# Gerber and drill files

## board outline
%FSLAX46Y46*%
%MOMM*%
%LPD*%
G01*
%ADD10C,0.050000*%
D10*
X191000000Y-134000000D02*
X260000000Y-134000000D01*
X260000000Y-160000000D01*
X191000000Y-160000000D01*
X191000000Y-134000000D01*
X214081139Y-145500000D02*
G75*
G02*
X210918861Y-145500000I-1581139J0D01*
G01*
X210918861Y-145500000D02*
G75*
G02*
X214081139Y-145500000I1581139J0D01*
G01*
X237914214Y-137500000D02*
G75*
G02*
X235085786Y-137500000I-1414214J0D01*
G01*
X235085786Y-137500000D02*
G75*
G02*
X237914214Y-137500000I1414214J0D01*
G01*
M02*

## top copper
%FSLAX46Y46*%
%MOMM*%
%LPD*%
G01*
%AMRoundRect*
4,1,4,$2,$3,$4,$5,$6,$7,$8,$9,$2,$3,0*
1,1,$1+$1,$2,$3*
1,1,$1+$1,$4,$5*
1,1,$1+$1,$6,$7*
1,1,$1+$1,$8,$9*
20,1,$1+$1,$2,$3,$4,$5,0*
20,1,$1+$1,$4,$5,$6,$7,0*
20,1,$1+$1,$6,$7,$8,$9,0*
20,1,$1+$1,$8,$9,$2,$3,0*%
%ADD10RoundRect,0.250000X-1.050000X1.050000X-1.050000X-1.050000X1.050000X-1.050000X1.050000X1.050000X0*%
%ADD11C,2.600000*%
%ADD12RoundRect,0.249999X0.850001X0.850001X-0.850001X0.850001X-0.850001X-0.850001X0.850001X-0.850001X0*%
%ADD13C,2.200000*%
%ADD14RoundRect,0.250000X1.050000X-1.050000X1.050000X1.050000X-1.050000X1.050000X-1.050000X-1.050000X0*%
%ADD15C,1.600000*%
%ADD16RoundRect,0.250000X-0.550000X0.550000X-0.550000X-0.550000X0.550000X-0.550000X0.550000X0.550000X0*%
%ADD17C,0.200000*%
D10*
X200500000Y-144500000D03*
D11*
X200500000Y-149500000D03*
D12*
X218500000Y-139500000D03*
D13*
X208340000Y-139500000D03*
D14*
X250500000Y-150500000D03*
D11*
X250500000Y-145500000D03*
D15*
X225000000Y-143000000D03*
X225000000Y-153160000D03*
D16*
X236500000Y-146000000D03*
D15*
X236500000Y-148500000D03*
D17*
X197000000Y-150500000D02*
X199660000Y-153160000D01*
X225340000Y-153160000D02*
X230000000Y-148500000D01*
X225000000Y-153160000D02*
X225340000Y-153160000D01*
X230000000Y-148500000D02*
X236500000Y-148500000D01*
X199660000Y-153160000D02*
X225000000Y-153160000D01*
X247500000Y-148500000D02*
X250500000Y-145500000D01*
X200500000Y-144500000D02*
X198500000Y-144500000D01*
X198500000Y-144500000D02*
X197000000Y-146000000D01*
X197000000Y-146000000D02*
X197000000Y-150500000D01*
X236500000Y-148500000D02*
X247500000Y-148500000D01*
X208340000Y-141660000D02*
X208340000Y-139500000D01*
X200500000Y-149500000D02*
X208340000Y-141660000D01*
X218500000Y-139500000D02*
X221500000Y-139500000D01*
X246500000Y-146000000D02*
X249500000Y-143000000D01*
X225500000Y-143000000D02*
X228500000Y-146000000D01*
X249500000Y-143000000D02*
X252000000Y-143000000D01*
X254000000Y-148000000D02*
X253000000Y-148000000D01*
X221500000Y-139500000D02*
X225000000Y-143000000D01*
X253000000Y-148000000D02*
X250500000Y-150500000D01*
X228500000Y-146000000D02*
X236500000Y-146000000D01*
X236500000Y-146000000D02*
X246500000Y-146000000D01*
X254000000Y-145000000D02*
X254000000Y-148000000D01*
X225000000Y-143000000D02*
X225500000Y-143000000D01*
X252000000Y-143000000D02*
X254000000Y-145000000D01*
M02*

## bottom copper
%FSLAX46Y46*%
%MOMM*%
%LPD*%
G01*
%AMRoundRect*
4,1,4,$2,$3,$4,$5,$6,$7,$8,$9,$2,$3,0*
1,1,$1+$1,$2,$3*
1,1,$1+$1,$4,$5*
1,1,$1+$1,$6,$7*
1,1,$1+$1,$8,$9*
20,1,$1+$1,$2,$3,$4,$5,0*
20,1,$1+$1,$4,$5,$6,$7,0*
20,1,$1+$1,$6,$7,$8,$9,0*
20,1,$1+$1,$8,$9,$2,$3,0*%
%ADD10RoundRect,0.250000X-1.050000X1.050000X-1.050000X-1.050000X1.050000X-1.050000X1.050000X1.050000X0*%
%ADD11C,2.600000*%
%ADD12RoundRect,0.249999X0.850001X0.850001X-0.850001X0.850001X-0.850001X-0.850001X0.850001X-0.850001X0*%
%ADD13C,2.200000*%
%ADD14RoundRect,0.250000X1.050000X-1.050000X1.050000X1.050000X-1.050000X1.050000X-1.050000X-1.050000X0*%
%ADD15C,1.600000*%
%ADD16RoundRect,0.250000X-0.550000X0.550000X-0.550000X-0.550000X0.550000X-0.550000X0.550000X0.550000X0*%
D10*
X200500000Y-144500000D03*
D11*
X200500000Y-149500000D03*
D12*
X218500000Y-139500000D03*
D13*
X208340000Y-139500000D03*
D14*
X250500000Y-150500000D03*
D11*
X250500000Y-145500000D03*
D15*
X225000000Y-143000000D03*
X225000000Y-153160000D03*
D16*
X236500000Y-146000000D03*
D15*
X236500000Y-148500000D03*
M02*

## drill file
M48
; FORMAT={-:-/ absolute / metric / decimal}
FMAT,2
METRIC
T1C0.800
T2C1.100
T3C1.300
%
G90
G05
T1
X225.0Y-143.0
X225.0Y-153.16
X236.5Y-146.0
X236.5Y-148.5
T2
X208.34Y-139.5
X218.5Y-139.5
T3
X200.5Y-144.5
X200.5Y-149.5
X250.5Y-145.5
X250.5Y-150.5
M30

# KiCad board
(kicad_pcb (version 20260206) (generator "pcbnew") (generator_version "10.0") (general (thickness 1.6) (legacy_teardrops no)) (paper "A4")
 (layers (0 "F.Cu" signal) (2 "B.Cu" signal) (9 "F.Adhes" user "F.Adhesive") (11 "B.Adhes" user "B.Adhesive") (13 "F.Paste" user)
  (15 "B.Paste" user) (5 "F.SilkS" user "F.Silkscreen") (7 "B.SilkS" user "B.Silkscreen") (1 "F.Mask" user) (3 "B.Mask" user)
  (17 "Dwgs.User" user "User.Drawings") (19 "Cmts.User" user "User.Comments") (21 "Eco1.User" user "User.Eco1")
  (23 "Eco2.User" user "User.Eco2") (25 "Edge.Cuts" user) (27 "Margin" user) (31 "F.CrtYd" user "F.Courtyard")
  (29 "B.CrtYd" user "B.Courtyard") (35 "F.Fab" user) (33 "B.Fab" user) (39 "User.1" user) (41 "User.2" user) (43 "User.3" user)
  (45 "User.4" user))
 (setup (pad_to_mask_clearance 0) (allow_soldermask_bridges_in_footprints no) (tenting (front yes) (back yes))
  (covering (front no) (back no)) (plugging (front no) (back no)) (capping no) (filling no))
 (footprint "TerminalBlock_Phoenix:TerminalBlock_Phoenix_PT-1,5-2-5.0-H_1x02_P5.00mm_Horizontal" (layer "F.Cu") (at 200.5 144.5 -90)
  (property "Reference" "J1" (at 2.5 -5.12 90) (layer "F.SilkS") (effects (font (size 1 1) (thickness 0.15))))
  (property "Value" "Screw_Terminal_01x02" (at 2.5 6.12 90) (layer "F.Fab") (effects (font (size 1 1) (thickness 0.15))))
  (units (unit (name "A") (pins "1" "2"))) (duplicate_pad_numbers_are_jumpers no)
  (pad "1" thru_hole roundrect (at 0 0 270) (size 2.6 2.6) (drill 1.3) (layers "*.Cu" "*.Mask") (remove_unused_layers no)
   (roundrect_rratio 0.096154) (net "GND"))
  (pad "2" thru_hole circle (at 5 0 270) (size 2.6 2.6) (drill 1.3) (layers "*.Cu" "*.Mask") (remove_unused_layers no) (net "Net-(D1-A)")))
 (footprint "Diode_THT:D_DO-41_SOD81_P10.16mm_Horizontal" (layer "F.Cu") (at 218.5 139.5 180)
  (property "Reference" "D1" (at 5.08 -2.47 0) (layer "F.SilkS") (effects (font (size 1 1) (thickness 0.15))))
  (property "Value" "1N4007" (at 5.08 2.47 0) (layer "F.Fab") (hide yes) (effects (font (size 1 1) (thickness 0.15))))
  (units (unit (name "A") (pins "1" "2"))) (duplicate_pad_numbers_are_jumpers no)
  (pad "1" thru_hole roundrect (at 0 0 180) (size 2.2 2.2) (drill 1.1) (layers "*.Cu" "*.Mask") (remove_unused_layers no)
   (roundrect_rratio 0.113636) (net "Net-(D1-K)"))
  (pad "2" thru_hole circle (at 10.16 0 180) (size 2.2 2.2) (drill 1.1) (layers "*.Cu" "*.Mask") (remove_unused_layers no)
   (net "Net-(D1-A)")))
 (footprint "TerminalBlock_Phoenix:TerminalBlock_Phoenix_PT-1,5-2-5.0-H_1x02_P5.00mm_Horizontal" (layer "F.Cu") (at 250.5 150.5 90)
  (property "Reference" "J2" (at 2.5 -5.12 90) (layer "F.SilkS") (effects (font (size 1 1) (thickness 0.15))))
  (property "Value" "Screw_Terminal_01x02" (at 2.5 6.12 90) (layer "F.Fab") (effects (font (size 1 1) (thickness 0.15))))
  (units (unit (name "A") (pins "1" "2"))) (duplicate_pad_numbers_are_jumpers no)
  (pad "1" thru_hole roundrect (at 0 0 90) (size 2.6 2.6) (drill 1.3) (layers "*.Cu" "*.Mask") (remove_unused_layers no)
   (roundrect_rratio 0.096154) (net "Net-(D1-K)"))
  (pad "2" thru_hole circle (at 5 0 90) (size 2.6 2.6) (drill 1.3) (layers "*.Cu" "*.Mask") (remove_unused_layers no) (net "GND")))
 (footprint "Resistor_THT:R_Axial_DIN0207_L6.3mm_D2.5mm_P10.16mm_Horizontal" (layer "F.Cu") (at 225 143 -90)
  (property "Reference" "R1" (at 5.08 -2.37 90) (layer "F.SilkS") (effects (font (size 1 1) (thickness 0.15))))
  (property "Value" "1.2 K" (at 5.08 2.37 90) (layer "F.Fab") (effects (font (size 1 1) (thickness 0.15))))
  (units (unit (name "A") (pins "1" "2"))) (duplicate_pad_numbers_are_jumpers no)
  (pad "1" thru_hole circle (at 0 0 270) (size 1.6 1.6) (drill 0.8) (layers "*.Cu" "*.Mask") (remove_unused_layers no) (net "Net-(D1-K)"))
  (pad "2" thru_hole circle (at 10.16 0 270) (size 1.6 1.6) (drill 0.8) (layers "*.Cu" "*.Mask") (remove_unused_layers no) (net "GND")))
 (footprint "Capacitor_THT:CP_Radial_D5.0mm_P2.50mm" (layer "F.Cu") (at 236.5 146 -90)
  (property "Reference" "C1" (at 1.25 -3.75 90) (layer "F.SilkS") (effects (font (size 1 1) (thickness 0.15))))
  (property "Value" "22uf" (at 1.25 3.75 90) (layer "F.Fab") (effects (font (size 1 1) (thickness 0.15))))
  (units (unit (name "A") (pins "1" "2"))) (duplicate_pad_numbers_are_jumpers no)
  (pad "1" thru_hole roundrect (at 0 0 270) (size 1.6 1.6) (drill 0.8) (layers "*.Cu" "*.Mask") (remove_unused_layers no)
   (roundrect_rratio 0.15625) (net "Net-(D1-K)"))
  (pad "2" thru_hole circle (at 2.5 0 270) (size 1.6 1.6) (drill 0.8) (layers "*.Cu" "*.Mask") (remove_unused_layers no) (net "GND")))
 (gr_rect (start 191 134) (end 260 160) (stroke (width 0.05) (type default)) (fill no) (layer "Edge.Cuts"))
 (gr_circle (center 212.5 145.5) (end 214 146) (stroke (width 0.05) (type default)) (fill no) (layer "Edge.Cuts"))
 (gr_circle (center 236.5 137.5) (end 237.5 138.5) (stroke (width 0.05) (type default)) (fill no) (layer "Edge.Cuts"))
 (segment (start 197 150.5) (end 199.66 153.16) (width 0.2) (layer "F.Cu") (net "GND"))
 (segment (start 225.34 153.16) (end 230 148.5) (width 0.2) (layer "F.Cu") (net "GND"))
 (segment (start 225 153.16) (end 225.34 153.16) (width 0.2) (layer "F.Cu") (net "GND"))
 (segment (start 230 148.5) (end 236.5 148.5) (width 0.2) (layer "F.Cu") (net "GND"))
 (segment (start 199.66 153.16) (end 225 153.16) (width 0.2) (layer "F.Cu") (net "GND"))
 (segment (start 247.5 148.5) (end 250.5 145.5) (width 0.2) (layer "F.Cu") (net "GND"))
 (segment (start 200.5 144.5) (end 198.5 144.5) (width 0.2) (layer "F.Cu") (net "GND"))
 (segment (start 198.5 144.5) (end 197 146) (width 0.2) (layer "F.Cu") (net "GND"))
 (segment (start 197 146) (end 197 150.5) (width 0.2) (layer "F.Cu") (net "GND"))
 (segment (start 236.5 148.5) (end 247.5 148.5) (width 0.2) (layer "F.Cu") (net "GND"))
 (segment (start 208.34 141.66) (end 208.34 139.5) (width 0.2) (layer "F.Cu") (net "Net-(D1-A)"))
 (segment (start 200.5 149.5) (end 208.34 141.66) (width 0.2) (layer "F.Cu") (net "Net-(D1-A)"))
 (segment (start 218.5 139.5) (end 221.5 139.5) (width 0.2) (layer "F.Cu") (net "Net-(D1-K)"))
 (segment (start 246.5 146) (end 249.5 143) (width 0.2) (layer "F.Cu") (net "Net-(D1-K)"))
 (segment (start 225.5 143) (end 228.5 146) (width 0.2) (layer "F.Cu") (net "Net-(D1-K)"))
 (segment (start 249.5 143) (end 252 143) (width 0.2) (layer "F.Cu") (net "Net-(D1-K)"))
 (segment (start 254 148) (end 253 148) (width 0.2) (layer "F.Cu") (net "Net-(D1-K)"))
 (segment (start 221.5 139.5) (end 225 143) (width 0.2) (layer "F.Cu") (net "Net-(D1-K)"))
 (segment (start 253 148) (end 250.5 150.5) (width 0.2) (layer "F.Cu") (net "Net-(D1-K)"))
 (segment (start 228.5 146) (end 236.5 146) (width 0.2) (layer "F.Cu") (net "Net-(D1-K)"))
 (segment (start 236.5 146) (end 246.5 146) (width 0.2) (layer "F.Cu") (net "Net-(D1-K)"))
 (segment (start 254 145) (end 254 148) (width 0.2) (layer "F.Cu") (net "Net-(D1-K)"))
 (segment (start 225 143) (end 225.5 143) (width 0.2) (layer "F.Cu") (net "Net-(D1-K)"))
 (segment (start 252 143) (end 254 145) (width 0.2) (layer "F.Cu") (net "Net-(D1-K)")))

